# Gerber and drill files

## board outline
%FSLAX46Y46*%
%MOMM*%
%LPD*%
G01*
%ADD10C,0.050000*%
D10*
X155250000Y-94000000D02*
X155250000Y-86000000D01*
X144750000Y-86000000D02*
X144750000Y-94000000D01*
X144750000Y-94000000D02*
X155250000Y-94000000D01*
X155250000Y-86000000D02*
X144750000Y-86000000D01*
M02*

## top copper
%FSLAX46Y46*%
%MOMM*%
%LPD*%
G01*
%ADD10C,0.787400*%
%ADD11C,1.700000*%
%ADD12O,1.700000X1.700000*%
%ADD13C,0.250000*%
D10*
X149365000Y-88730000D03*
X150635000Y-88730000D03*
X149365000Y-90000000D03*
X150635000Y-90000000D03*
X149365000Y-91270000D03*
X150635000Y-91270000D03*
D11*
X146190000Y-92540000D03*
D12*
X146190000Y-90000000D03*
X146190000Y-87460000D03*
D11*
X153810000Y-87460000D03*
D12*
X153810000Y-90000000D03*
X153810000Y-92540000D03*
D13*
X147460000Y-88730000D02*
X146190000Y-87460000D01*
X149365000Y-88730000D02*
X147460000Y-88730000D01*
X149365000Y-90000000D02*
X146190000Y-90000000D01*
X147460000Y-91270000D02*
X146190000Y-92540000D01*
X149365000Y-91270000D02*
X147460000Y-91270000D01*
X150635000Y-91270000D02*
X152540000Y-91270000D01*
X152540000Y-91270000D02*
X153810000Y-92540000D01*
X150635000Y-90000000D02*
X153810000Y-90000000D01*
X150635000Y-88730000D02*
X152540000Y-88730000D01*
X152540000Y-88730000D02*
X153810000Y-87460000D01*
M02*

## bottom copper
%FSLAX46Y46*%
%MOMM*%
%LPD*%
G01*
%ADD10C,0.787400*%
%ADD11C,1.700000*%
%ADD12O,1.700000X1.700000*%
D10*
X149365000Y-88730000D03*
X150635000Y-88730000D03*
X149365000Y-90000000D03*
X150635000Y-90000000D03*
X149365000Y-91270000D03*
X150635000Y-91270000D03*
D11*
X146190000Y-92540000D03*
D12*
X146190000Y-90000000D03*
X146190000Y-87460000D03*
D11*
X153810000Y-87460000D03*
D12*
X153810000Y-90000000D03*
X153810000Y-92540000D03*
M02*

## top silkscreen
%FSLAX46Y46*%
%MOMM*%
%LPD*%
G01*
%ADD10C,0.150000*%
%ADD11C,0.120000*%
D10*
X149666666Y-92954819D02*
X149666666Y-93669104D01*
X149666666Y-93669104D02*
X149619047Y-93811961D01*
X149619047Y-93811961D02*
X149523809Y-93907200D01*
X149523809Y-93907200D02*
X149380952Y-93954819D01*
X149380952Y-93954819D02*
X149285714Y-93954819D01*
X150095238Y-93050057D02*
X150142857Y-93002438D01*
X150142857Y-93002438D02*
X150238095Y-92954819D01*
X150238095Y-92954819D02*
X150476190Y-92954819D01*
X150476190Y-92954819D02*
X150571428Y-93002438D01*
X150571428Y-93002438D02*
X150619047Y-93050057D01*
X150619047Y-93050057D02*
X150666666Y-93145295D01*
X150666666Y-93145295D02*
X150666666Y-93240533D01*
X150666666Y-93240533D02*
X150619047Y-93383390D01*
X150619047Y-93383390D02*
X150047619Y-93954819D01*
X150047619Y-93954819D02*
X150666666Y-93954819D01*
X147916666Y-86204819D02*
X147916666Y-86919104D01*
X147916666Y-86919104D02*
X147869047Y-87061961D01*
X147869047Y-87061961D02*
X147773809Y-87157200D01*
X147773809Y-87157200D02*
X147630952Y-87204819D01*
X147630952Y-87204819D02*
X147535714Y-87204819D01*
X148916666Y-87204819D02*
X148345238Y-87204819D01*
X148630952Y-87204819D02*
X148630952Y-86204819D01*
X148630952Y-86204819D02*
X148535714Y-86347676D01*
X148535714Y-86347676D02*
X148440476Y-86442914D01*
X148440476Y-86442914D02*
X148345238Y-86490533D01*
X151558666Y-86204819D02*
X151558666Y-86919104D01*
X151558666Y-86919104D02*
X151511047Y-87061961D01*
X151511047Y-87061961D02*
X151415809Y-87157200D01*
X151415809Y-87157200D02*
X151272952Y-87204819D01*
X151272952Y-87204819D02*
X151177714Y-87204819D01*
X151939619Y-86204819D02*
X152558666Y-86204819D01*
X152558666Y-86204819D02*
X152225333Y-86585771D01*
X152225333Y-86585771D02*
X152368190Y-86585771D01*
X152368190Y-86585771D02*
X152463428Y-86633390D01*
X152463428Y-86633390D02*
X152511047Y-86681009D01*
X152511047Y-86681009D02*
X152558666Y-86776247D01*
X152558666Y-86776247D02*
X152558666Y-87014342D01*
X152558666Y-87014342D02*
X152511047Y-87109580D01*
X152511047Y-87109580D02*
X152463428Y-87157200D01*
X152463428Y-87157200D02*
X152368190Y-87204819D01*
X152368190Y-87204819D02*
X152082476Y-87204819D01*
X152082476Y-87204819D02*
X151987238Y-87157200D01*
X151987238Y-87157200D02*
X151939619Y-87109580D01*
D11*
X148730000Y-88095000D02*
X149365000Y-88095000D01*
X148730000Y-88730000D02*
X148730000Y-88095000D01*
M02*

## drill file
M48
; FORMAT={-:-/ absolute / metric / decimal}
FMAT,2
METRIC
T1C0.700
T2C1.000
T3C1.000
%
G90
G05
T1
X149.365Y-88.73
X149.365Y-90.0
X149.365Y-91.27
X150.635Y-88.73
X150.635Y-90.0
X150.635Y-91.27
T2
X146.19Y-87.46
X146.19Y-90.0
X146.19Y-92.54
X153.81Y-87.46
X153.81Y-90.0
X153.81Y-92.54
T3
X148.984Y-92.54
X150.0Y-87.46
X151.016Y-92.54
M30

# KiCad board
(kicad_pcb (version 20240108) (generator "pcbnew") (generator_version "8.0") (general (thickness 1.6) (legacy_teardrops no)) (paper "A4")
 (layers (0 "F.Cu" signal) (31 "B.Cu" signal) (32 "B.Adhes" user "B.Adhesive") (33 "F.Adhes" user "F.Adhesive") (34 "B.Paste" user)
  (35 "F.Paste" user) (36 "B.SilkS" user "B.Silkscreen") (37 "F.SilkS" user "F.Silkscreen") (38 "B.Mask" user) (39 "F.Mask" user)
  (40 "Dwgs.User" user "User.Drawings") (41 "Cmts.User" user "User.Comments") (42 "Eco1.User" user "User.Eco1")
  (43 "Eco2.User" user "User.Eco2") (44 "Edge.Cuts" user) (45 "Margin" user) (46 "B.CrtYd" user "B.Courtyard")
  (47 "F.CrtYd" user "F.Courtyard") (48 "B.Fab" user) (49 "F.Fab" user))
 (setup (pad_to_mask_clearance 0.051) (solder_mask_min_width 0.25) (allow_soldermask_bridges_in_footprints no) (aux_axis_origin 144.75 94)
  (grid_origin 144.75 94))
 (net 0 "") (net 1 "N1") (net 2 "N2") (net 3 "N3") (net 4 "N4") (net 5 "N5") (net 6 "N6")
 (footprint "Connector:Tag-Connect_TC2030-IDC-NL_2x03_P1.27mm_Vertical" (layer "F.Cu") (at 150 90 -90)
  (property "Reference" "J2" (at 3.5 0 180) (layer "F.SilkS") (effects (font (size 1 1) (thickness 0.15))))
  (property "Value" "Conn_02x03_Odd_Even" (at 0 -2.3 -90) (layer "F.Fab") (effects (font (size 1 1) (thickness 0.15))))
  (fp_line (start -1.905 1.27) (end -1.905 0.635) (stroke (width 0.12) (type solid)) (layer "F.SilkS"))
  (fp_line (start -1.27 1.27) (end -1.905 1.27) (stroke (width 0.12) (type solid)) (layer "F.SilkS"))
  (pad "" np_thru_hole circle (at -2.54 0 270) (size 1 1) (drill 1) (layers "*.Cu" "*.Mask"))
  (pad "" np_thru_hole circle (at 2.54 -1.016 270) (size 1 1) (drill 1) (layers "*.Cu" "*.Mask"))
  (pad "" np_thru_hole circle (at 2.54 1.016 270) (size 1 1) (drill 1) (layers "*.Cu" "*.Mask"))
  (pad "1" thru_hole circle (at -1.27 0.635 270) (size 0.7874 0.7874) (drill 0.7) (layers "*.Cu" "*.Mask") (remove_unused_layers no)
   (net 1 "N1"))
  (pad "2" thru_hole circle (at -1.27 -0.635 270) (size 0.7874 0.7874) (drill 0.7) (layers "*.Cu" "*.Mask") (remove_unused_layers no)
   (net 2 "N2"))
  (pad "3" thru_hole circle (at 0 0.635 270) (size 0.7874 0.7874) (drill 0.7) (layers "*.Cu" "*.Mask") (remove_unused_layers no)
   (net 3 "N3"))
  (pad "4" thru_hole circle (at 0 -0.635 270) (size 0.7874 0.7874) (drill 0.7) (layers "*.Cu" "*.Mask") (remove_unused_layers no)
   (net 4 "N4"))
  (pad "5" thru_hole circle (at 1.27 0.635 270) (size 0.7874 0.7874) (drill 0.7) (layers "*.Cu" "*.Mask") (remove_unused_layers no)
   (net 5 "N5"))
  (pad "6" thru_hole circle (at 1.27 -0.635 270) (size 0.7874 0.7874) (drill 0.7) (layers "*.Cu" "*.Mask") (remove_unused_layers no)
   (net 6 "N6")))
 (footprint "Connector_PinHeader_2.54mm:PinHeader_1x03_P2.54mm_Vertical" (layer "B.Cu") (at 146.19 92.54)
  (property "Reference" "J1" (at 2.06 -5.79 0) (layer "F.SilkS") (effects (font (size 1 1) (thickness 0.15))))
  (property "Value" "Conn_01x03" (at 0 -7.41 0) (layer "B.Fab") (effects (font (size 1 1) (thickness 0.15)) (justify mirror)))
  (pad "1" thru_hole circle (at 0 0) (size 1.7 1.7) (drill 1) (layers "*.Cu" "*.Mask") (remove_unused_layers no) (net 5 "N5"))
  (pad "2" thru_hole oval (at 0 -2.54) (size 1.7 1.7) (drill 1) (layers "*.Cu" "*.Mask") (remove_unused_layers no) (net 3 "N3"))
  (pad "3" thru_hole oval (at 0 -5.08) (size 1.7 1.7) (drill 1) (layers "*.Cu" "*.Mask") (remove_unused_layers no) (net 1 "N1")))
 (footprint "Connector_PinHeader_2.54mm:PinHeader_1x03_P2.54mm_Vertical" (layer "B.Cu") (at 153.81 87.46 180)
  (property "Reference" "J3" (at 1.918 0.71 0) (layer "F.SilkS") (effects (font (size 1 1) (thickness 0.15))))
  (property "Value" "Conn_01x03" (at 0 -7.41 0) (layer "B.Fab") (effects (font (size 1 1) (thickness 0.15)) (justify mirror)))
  (pad "1" thru_hole circle (at 0 0 180) (size 1.7 1.7) (drill 1) (layers "*.Cu" "*.Mask") (remove_unused_layers no) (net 2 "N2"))
  (pad "2" thru_hole oval (at 0 -2.54 180) (size 1.7 1.7) (drill 1) (layers "*.Cu" "*.Mask") (remove_unused_layers no) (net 4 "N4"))
  (pad "3" thru_hole oval (at 0 -5.08 180) (size 1.7 1.7) (drill 1) (layers "*.Cu" "*.Mask") (remove_unused_layers no) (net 6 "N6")))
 (gr_line (start 155.25 94) (end 155.25 86) (stroke (width 0.05) (type solid)) (layer "Edge.Cuts"))
 (gr_line (start 144.75 86) (end 144.75 94) (stroke (width 0.05) (type solid)) (layer "Edge.Cuts"))
 (gr_line (start 144.75 94) (end 155.25 94) (stroke (width 0.05) (type solid)) (layer "Edge.Cuts"))
 (gr_line (start 155.25 86) (end 144.75 86) (stroke (width 0.05) (type solid)) (layer "Edge.Cuts"))
 (segment (start 147.46 88.73) (end 146.19 87.46) (width 0.25) (layer "F.Cu") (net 1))
 (segment (start 149.365 88.73) (end 147.46 88.73) (width 0.25) (layer "F.Cu") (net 1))
 (segment (start 149.365 90) (end 146.19 90) (width 0.25) (layer "F.Cu") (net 3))
 (segment (start 147.46 91.27) (end 146.19 92.54) (width 0.25) (layer "F.Cu") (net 5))
 (segment (start 149.365 91.27) (end 147.46 91.27) (width 0.25) (layer "F.Cu") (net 5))
 (segment (start 150.635 91.27) (end 152.54 91.27) (width 0.25) (layer "F.Cu") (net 6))
 (segment (start 152.54 91.27) (end 153.81 92.54) (width 0.25) (layer "F.Cu") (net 6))
 (segment (start 150.635 90) (end 153.81 90) (width 0.25) (layer "F.Cu") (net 4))
 (segment (start 150.635 88.73) (end 152.54 88.73) (width 0.25) (layer "F.Cu") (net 2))
 (segment (start 152.54 88.73) (end 153.81 87.46) (width 0.25) (layer "F.Cu") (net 2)))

